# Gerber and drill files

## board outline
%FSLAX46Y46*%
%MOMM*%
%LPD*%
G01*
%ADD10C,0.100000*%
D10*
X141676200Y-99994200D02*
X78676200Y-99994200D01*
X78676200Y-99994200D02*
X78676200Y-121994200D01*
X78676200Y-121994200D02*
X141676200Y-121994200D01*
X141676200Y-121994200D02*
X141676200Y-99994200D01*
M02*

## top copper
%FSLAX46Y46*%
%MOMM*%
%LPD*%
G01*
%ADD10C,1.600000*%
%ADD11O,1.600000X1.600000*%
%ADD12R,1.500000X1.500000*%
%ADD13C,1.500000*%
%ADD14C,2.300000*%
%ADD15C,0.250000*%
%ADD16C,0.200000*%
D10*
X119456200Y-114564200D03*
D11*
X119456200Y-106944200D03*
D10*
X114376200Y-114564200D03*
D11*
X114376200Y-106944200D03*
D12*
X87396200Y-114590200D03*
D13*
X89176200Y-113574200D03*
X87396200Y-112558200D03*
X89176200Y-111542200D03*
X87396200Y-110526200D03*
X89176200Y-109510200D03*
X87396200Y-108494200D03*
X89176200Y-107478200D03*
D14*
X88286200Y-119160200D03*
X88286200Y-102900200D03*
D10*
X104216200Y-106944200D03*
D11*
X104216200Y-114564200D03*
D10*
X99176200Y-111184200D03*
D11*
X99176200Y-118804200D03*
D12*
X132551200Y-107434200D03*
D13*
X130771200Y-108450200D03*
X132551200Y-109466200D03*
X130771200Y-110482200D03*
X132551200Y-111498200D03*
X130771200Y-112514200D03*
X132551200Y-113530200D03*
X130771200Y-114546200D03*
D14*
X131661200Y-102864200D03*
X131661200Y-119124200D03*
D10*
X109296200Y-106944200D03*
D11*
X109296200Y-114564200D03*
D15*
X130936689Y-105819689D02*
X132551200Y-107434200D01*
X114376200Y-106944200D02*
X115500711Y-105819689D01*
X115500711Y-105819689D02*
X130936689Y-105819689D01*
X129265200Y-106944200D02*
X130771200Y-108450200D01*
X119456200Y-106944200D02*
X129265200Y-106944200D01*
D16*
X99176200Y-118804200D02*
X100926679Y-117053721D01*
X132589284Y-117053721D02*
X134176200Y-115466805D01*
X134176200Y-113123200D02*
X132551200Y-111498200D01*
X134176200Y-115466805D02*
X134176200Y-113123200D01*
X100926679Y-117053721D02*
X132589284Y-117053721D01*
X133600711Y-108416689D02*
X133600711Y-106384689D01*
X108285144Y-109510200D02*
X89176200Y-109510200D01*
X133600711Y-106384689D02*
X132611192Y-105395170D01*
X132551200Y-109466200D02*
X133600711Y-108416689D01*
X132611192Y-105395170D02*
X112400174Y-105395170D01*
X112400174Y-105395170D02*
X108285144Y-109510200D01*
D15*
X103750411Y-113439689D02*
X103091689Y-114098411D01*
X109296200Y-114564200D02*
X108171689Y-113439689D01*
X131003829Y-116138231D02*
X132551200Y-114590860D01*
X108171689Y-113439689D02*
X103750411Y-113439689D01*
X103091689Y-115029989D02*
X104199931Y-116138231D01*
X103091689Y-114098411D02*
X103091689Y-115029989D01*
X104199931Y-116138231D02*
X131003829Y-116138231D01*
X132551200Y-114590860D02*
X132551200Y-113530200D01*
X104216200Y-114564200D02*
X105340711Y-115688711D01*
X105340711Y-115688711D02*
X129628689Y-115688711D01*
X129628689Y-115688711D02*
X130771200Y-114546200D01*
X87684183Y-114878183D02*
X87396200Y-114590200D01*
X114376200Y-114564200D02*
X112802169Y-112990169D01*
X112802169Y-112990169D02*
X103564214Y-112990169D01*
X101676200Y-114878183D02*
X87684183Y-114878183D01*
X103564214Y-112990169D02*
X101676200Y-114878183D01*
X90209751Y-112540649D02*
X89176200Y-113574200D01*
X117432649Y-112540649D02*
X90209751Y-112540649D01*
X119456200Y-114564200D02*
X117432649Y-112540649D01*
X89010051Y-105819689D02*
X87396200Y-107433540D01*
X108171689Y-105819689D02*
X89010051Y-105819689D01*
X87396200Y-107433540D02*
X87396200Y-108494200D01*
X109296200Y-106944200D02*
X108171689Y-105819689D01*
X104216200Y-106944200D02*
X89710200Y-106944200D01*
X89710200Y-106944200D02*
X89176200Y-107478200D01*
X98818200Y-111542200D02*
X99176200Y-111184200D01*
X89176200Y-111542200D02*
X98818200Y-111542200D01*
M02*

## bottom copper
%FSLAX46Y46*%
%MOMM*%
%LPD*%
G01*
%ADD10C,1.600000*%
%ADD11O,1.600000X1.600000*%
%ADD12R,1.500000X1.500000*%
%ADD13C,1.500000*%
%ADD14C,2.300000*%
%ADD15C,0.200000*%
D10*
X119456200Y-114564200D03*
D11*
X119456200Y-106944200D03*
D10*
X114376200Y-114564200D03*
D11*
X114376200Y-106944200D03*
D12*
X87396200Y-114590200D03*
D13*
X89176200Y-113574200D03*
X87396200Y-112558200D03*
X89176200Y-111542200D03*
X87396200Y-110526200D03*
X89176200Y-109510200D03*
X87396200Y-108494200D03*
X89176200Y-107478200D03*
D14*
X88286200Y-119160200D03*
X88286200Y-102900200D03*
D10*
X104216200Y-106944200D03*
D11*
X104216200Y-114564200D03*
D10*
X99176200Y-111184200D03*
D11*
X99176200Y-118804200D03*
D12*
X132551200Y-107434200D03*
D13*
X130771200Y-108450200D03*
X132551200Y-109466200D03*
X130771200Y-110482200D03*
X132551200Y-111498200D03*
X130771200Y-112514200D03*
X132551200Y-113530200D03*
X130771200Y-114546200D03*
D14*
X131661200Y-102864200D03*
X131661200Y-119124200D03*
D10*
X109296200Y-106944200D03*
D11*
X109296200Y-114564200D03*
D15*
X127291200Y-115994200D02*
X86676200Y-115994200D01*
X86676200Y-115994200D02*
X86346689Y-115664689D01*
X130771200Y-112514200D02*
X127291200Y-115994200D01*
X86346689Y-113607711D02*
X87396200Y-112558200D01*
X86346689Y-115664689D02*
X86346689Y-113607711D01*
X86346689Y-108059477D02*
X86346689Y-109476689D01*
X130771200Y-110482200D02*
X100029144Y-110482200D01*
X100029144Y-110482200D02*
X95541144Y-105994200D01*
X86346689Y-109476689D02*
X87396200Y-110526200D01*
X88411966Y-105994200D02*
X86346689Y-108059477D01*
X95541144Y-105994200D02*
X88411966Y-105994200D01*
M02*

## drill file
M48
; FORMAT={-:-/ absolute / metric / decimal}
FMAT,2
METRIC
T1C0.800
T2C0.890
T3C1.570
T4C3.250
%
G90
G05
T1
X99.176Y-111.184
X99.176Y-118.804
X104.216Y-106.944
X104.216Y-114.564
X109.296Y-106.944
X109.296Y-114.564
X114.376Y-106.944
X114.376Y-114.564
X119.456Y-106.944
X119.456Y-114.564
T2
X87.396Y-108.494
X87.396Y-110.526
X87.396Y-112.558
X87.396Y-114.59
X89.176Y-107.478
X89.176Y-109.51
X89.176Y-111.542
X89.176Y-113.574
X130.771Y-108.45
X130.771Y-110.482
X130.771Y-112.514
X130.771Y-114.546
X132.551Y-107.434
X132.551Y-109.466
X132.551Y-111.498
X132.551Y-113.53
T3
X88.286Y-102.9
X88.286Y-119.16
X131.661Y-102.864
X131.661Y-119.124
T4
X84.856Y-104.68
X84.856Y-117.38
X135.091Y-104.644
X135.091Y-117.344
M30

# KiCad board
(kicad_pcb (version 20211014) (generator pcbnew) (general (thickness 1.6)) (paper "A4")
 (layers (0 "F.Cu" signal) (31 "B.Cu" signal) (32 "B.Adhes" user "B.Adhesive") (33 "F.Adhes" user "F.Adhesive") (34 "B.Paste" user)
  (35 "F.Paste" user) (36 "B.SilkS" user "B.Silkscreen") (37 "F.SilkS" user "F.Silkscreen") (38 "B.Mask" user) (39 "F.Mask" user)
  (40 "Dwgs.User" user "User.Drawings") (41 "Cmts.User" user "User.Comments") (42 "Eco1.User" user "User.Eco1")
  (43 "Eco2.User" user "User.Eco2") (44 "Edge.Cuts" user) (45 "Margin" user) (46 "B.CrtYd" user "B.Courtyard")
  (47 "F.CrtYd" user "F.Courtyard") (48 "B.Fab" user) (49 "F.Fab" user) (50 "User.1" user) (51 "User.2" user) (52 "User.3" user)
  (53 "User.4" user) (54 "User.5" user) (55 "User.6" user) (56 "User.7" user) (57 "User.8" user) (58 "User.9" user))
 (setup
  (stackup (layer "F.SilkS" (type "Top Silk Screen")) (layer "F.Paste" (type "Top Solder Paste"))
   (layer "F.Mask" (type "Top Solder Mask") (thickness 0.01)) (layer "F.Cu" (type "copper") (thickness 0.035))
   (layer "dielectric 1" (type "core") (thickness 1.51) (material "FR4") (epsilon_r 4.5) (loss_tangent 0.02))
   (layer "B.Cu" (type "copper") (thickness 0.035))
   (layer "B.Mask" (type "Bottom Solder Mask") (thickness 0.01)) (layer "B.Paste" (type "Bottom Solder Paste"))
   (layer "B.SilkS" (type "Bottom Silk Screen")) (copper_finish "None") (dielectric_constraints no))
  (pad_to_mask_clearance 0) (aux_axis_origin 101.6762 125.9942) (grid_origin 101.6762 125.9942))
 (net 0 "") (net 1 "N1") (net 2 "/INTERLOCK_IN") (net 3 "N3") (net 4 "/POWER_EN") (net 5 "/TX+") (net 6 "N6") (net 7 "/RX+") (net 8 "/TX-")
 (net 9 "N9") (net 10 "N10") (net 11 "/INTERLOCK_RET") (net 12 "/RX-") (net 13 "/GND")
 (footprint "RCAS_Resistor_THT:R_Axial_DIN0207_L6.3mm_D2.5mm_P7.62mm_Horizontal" (layer "F.Cu") (at 119.4562 114.5642 90)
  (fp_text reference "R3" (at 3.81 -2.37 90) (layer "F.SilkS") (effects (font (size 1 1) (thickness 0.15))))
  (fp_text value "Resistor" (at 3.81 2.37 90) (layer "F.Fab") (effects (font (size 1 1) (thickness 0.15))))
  (pad "1" thru_hole circle locked (at 0 0 90) (size 1.6 1.6) (drill 0.8) (layers *.Cu *.Mask) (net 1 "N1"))
  (pad "2" thru_hole oval locked (at 7.62 0 90) (size 1.6 1.6) (drill 0.8) (layers *.Cu *.Mask) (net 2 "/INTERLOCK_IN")))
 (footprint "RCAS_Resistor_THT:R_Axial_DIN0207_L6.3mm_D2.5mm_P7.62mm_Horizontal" (layer "F.Cu") (at 114.3762 114.5642 90)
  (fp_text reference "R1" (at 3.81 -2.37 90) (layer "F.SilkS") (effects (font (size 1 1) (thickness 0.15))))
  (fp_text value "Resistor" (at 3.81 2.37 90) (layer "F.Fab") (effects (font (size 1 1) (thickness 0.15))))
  (pad "1" thru_hole circle locked (at 0 0 90) (size 1.6 1.6) (drill 0.8) (layers *.Cu *.Mask) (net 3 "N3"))
  (pad "2" thru_hole oval locked (at 7.62 0 90) (size 1.6 1.6) (drill 0.8) (layers *.Cu *.Mask) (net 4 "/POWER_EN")))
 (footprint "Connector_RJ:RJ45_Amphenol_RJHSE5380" (layer "F.Cu") (at 87.3962 114.5902 90)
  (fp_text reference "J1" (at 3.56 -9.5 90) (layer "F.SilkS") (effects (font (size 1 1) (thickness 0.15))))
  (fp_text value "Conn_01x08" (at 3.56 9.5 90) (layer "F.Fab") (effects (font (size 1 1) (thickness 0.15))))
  (pad "" np_thru_hole circle (at 9.91 -2.54 90) (size 3.25 3.25) (drill 3.25) (layers *.Cu *.Mask))
  (pad "" np_thru_hole circle (at -2.79 -2.54 90) (size 3.25 3.25) (drill 3.25) (layers *.Cu *.Mask))
  (pad "1" thru_hole rect (at 0 0 90) (size 1.5 1.5) (drill 0.89) (layers *.Cu *.Mask) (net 3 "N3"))
  (pad "2" thru_hole circle (at 1.016 1.78 90) (size 1.5 1.5) (drill 0.89) (layers *.Cu *.Mask) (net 1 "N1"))
  (pad "3" thru_hole circle (at 2.032 0 90) (size 1.5 1.5) (drill 0.89) (layers *.Cu *.Mask) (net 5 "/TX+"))
  (pad "4" thru_hole circle (at 3.048 1.78 90) (size 1.5 1.5) (drill 0.89) (layers *.Cu *.Mask) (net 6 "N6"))
  (pad "5" thru_hole circle (at 4.064 0 90) (size 1.5 1.5) (drill 0.89) (layers *.Cu *.Mask) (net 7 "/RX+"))
  (pad "6" thru_hole circle (at 5.08 1.78 90) (size 1.5 1.5) (drill 0.89) (layers *.Cu *.Mask) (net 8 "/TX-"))
  (pad "7" thru_hole circle (at 6.096 0 90) (size 1.5 1.5) (drill 0.89) (layers *.Cu *.Mask) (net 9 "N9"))
  (pad "8" thru_hole circle (at 7.112 1.78 90) (size 1.5 1.5) (drill 0.89) (layers *.Cu *.Mask) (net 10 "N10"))
  (pad "SH" thru_hole circle (at -4.57 0.89 90) (size 2.3 2.3) (drill 1.57) (layers *.Cu *.Mask))
  (pad "SH" thru_hole circle (at 11.69 0.89 90) (size 2.3 2.3) (drill 1.57) (layers *.Cu *.Mask)))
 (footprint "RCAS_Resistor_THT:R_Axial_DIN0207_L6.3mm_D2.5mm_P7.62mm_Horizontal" (layer "F.Cu") (at 104.2162 106.9442 -90)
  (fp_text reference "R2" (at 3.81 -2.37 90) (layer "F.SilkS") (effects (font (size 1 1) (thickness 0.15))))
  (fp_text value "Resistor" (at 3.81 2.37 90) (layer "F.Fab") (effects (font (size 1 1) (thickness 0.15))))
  (pad "1" thru_hole circle locked (at 0 0 270) (size 1.6 1.6) (drill 0.8) (layers *.Cu *.Mask) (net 10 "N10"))
  (pad "2" thru_hole oval locked (at 7.62 0 270) (size 1.6 1.6) (drill 0.8) (layers *.Cu *.Mask) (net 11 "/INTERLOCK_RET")))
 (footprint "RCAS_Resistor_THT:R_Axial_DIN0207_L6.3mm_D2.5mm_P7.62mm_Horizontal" (layer "F.Cu") (at 99.1762 111.1842 -90)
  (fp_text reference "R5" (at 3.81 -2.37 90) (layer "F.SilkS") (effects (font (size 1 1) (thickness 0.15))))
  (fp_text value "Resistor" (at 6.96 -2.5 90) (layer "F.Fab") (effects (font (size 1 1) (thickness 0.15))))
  (pad "1" thru_hole circle locked (at 0 0 270) (size 1.6 1.6) (drill 0.8) (layers *.Cu *.Mask) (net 6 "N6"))
  (pad "2" thru_hole oval locked (at 7.62 0 270) (size 1.6 1.6) (drill 0.8) (layers *.Cu *.Mask) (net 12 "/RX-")))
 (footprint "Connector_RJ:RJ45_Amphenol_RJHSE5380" (layer "F.Cu") (at 132.5512 107.4342 -90)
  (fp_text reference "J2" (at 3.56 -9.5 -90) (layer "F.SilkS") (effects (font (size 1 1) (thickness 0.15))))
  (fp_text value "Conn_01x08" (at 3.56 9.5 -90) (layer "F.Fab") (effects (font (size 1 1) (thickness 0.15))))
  (pad "" np_thru_hole circle (at 9.91 -2.54 270) (size 3.25 3.25) (drill 3.25) (layers *.Cu *.Mask))
  (pad "" np_thru_hole circle (at -2.79 -2.54 270) (size 3.25 3.25) (drill 3.25) (layers *.Cu *.Mask))
  (pad "1" thru_hole rect (at 0 0 270) (size 1.5 1.5) (drill 0.89) (layers *.Cu *.Mask) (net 4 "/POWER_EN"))
  (pad "2" thru_hole circle (at 1.016 1.78 270) (size 1.5 1.5) (drill 0.89) (layers *.Cu *.Mask) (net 2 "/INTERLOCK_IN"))
  (pad "3" thru_hole circle (at 2.032 0 270) (size 1.5 1.5) (drill 0.89) (layers *.Cu *.Mask) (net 8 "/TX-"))
  (pad "4" thru_hole circle (at 3.048 1.78 270) (size 1.5 1.5) (drill 0.89) (layers *.Cu *.Mask) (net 7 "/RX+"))
  (pad "5" thru_hole circle (at 4.064 0 270) (size 1.5 1.5) (drill 0.89) (layers *.Cu *.Mask) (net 12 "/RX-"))
  (pad "6" thru_hole circle (at 5.08 1.78 270) (size 1.5 1.5) (drill 0.89) (layers *.Cu *.Mask) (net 5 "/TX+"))
  (pad "7" thru_hole circle (at 6.096 0 270) (size 1.5 1.5) (drill 0.89) (layers *.Cu *.Mask) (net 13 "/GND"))
  (pad "8" thru_hole circle (at 7.112 1.78 270) (size 1.5 1.5) (drill 0.89) (layers *.Cu *.Mask) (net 11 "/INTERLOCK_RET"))
  (pad "SH" thru_hole circle (at -4.57 0.89 270) (size 2.3 2.3) (drill 1.57) (layers *.Cu *.Mask))
  (pad "SH" thru_hole circle (at 11.69 0.89 270) (size 2.3 2.3) (drill 1.57) (layers *.Cu *.Mask)))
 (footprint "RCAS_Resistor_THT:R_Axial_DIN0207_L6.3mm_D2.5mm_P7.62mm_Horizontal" (layer "F.Cu") (at 109.2962 106.9442 -90)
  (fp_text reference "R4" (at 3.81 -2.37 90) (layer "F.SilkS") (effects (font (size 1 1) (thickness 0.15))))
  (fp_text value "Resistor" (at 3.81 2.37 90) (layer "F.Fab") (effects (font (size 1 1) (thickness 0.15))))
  (pad "1" thru_hole circle locked (at 0 0 270) (size 1.6 1.6) (drill 0.8) (layers *.Cu *.Mask) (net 9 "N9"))
  (pad "2" thru_hole oval locked (at 7.62 0 270) (size 1.6 1.6) (drill 0.8) (layers *.Cu *.Mask) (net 13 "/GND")))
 (gr_line (start 141.6762 99.9942) (end 78.6762 99.9942) (layer "Edge.Cuts") (width 0.1))
 (gr_line (start 78.6762 99.9942) (end 78.6762 121.9942) (layer "Edge.Cuts") (width 0.1))
 (gr_line (start 78.6762 121.9942) (end 141.6762 121.9942) (layer "Edge.Cuts") (width 0.1))
 (gr_line (start 141.6762 121.9942) (end 141.6762 99.9942) (layer "Edge.Cuts") (width 0.1))
 (segment (start 130.936689 105.819689) (end 132.5512 107.4342) (width 0.25) (layer "F.Cu") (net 4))
 (segment (start 114.3762 106.9442) (end 115.500711 105.819689) (width 0.25) (layer "F.Cu") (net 4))
 (segment (start 115.500711 105.819689) (end 130.936689 105.819689) (width 0.25) (layer "F.Cu") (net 4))
 (segment (start 129.2652 106.9442) (end 130.7712 108.4502) (width 0.25) (layer "F.Cu") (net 2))
 (segment (start 119.4562 106.9442) (end 129.2652 106.9442) (width 0.25) (layer "F.Cu") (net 2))
 (segment (start 127.2912 115.9942) (end 86.6762 115.9942) (width 0.2) (layer "B.Cu") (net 5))
 (segment (start 86.6762 115.9942) (end 86.346689 115.664689) (width 0.2) (layer "B.Cu") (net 5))
 (segment (start 130.7712 112.5142) (end 127.2912 115.9942) (width 0.2) (layer "B.Cu") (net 5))
 (segment (start 86.346689 113.607711) (end 87.3962 112.5582) (width 0.2) (layer "B.Cu") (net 5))
 (segment (start 86.346689 115.664689) (end 86.346689 113.607711) (width 0.2) (layer "B.Cu") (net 5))
 (segment (start 99.1762 118.8042) (end 100.926679 117.053721) (width 0.2) (layer "F.Cu") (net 12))
 (segment (start 132.589284 117.053721) (end 134.1762 115.466805) (width 0.2) (layer "F.Cu") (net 12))
 (segment (start 134.1762 113.1232) (end 132.5512 111.4982) (width 0.2) (layer "F.Cu") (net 12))
 (segment (start 134.1762 115.466805) (end 134.1762 113.1232) (width 0.2) (layer "F.Cu") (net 12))
 (segment (start 100.926679 117.053721) (end 132.589284 117.053721) (width 0.2) (layer "F.Cu") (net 12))
 (segment (start 86.346689 108.059477) (end 86.346689 109.476689) (width 0.2) (layer "B.Cu") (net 7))
 (segment (start 130.7712 110.4822) (end 100.029144 110.4822) (width 0.2) (layer "B.Cu") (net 7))
 (segment (start 100.029144 110.4822) (end 95.541144 105.9942) (width 0.2) (layer "B.Cu") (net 7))
 (segment (start 86.346689 109.476689) (end 87.3962 110.5262) (width 0.2) (layer "B.Cu") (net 7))
 (segment (start 88.411966 105.9942) (end 86.346689 108.059477) (width 0.2) (layer "B.Cu") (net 7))
 (segment (start 95.541144 105.9942) (end 88.411966 105.9942) (width 0.2) (layer "B.Cu") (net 7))
 (segment (start 133.600711 108.416689) (end 133.600711 106.384689) (width 0.2) (layer "F.Cu") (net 8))
 (segment (start 108.285144 109.5102) (end 89.1762 109.5102) (width 0.2) (layer "F.Cu") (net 8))
 (segment (start 133.600711 106.384689) (end 132.611192 105.39517) (width 0.2) (layer "F.Cu") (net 8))
 (segment (start 132.5512 109.4662) (end 133.600711 108.416689) (width 0.2) (layer "F.Cu") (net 8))
 (segment (start 132.611192 105.39517) (end 112.400174 105.39517) (width 0.2) (layer "F.Cu") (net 8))
 (segment (start 112.400174 105.39517) (end 108.285144 109.5102) (width 0.2) (layer "F.Cu") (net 8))
 (segment (start 103.750411 113.439689) (end 103.091689 114.098411) (width 0.25) (layer "F.Cu") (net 13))
 (segment (start 109.2962 114.5642) (end 108.171689 113.439689) (width 0.25) (layer "F.Cu") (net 13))
 (segment (start 131.003829 116.138231) (end 132.5512 114.59086) (width 0.25) (layer "F.Cu") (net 13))
 (segment (start 108.171689 113.439689) (end 103.750411 113.439689) (width 0.25) (layer "F.Cu") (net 13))
 (segment (start 103.091689 115.029989) (end 104.199931 116.138231) (width 0.25) (layer "F.Cu") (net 13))
 (segment (start 103.091689 114.098411) (end 103.091689 115.029989) (width 0.25) (layer "F.Cu") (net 13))
 (segment (start 104.199931 116.138231) (end 131.003829 116.138231) (width 0.25) (layer "F.Cu") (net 13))
 (segment (start 132.5512 114.59086) (end 132.5512 113.5302) (width 0.25) (layer "F.Cu") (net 13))
 (segment (start 104.2162 114.5642) (end 105.340711 115.688711) (width 0.25) (layer "F.Cu") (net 11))
 (segment (start 105.340711 115.688711) (end 129.628689 115.688711) (width 0.25) (layer "F.Cu") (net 11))
 (segment (start 129.628689 115.688711) (end 130.7712 114.5462) (width 0.25) (layer "F.Cu") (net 11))
 (segment (start 87.684183 114.878183) (end 87.3962 114.5902) (width 0.25) (layer "F.Cu") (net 3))
 (segment (start 114.3762 114.5642) (end 112.802169 112.990169) (width 0.25) (layer "F.Cu") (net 3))
 (segment (start 112.802169 112.990169) (end 103.564214 112.990169) (width 0.25) (layer "F.Cu") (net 3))
 (segment (start 101.6762 114.878183) (end 87.684183 114.878183) (width 0.25) (layer "F.Cu") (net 3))
 (segment (start 103.564214 112.990169) (end 101.6762 114.878183) (width 0.25) (layer "F.Cu") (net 3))
 (segment (start 90.209751 112.540649) (end 89.1762 113.5742) (width 0.25) (layer "F.Cu") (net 1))
 (segment (start 117.432649 112.540649) (end 90.209751 112.540649) (width 0.25) (layer "F.Cu") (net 1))
 (segment (start 119.4562 114.5642) (end 117.432649 112.540649) (width 0.25) (layer "F.Cu") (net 1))
 (segment (start 89.010051 105.819689) (end 87.3962 107.43354) (width 0.25) (layer "F.Cu") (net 9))
 (segment (start 108.171689 105.819689) (end 89.010051 105.819689) (width 0.25) (layer "F.Cu") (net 9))
 (segment (start 87.3962 107.43354) (end 87.3962 108.4942) (width 0.25) (layer "F.Cu") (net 9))
 (segment (start 109.2962 106.9442) (end 108.171689 105.819689) (width 0.25) (layer "F.Cu") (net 9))
 (segment (start 104.2162 106.9442) (end 89.7102 106.9442) (width 0.25) (layer "F.Cu") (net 10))
 (segment (start 89.7102 106.9442) (end 89.1762 107.4782) (width 0.25) (layer "F.Cu") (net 10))
 (segment (start 98.8182 111.5422) (end 99.1762 111.1842) (width 0.25) (layer "F.Cu") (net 6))
 (segment (start 89.1762 111.5422) (end 98.8182 111.5422) (width 0.25) (layer "F.Cu") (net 6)))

